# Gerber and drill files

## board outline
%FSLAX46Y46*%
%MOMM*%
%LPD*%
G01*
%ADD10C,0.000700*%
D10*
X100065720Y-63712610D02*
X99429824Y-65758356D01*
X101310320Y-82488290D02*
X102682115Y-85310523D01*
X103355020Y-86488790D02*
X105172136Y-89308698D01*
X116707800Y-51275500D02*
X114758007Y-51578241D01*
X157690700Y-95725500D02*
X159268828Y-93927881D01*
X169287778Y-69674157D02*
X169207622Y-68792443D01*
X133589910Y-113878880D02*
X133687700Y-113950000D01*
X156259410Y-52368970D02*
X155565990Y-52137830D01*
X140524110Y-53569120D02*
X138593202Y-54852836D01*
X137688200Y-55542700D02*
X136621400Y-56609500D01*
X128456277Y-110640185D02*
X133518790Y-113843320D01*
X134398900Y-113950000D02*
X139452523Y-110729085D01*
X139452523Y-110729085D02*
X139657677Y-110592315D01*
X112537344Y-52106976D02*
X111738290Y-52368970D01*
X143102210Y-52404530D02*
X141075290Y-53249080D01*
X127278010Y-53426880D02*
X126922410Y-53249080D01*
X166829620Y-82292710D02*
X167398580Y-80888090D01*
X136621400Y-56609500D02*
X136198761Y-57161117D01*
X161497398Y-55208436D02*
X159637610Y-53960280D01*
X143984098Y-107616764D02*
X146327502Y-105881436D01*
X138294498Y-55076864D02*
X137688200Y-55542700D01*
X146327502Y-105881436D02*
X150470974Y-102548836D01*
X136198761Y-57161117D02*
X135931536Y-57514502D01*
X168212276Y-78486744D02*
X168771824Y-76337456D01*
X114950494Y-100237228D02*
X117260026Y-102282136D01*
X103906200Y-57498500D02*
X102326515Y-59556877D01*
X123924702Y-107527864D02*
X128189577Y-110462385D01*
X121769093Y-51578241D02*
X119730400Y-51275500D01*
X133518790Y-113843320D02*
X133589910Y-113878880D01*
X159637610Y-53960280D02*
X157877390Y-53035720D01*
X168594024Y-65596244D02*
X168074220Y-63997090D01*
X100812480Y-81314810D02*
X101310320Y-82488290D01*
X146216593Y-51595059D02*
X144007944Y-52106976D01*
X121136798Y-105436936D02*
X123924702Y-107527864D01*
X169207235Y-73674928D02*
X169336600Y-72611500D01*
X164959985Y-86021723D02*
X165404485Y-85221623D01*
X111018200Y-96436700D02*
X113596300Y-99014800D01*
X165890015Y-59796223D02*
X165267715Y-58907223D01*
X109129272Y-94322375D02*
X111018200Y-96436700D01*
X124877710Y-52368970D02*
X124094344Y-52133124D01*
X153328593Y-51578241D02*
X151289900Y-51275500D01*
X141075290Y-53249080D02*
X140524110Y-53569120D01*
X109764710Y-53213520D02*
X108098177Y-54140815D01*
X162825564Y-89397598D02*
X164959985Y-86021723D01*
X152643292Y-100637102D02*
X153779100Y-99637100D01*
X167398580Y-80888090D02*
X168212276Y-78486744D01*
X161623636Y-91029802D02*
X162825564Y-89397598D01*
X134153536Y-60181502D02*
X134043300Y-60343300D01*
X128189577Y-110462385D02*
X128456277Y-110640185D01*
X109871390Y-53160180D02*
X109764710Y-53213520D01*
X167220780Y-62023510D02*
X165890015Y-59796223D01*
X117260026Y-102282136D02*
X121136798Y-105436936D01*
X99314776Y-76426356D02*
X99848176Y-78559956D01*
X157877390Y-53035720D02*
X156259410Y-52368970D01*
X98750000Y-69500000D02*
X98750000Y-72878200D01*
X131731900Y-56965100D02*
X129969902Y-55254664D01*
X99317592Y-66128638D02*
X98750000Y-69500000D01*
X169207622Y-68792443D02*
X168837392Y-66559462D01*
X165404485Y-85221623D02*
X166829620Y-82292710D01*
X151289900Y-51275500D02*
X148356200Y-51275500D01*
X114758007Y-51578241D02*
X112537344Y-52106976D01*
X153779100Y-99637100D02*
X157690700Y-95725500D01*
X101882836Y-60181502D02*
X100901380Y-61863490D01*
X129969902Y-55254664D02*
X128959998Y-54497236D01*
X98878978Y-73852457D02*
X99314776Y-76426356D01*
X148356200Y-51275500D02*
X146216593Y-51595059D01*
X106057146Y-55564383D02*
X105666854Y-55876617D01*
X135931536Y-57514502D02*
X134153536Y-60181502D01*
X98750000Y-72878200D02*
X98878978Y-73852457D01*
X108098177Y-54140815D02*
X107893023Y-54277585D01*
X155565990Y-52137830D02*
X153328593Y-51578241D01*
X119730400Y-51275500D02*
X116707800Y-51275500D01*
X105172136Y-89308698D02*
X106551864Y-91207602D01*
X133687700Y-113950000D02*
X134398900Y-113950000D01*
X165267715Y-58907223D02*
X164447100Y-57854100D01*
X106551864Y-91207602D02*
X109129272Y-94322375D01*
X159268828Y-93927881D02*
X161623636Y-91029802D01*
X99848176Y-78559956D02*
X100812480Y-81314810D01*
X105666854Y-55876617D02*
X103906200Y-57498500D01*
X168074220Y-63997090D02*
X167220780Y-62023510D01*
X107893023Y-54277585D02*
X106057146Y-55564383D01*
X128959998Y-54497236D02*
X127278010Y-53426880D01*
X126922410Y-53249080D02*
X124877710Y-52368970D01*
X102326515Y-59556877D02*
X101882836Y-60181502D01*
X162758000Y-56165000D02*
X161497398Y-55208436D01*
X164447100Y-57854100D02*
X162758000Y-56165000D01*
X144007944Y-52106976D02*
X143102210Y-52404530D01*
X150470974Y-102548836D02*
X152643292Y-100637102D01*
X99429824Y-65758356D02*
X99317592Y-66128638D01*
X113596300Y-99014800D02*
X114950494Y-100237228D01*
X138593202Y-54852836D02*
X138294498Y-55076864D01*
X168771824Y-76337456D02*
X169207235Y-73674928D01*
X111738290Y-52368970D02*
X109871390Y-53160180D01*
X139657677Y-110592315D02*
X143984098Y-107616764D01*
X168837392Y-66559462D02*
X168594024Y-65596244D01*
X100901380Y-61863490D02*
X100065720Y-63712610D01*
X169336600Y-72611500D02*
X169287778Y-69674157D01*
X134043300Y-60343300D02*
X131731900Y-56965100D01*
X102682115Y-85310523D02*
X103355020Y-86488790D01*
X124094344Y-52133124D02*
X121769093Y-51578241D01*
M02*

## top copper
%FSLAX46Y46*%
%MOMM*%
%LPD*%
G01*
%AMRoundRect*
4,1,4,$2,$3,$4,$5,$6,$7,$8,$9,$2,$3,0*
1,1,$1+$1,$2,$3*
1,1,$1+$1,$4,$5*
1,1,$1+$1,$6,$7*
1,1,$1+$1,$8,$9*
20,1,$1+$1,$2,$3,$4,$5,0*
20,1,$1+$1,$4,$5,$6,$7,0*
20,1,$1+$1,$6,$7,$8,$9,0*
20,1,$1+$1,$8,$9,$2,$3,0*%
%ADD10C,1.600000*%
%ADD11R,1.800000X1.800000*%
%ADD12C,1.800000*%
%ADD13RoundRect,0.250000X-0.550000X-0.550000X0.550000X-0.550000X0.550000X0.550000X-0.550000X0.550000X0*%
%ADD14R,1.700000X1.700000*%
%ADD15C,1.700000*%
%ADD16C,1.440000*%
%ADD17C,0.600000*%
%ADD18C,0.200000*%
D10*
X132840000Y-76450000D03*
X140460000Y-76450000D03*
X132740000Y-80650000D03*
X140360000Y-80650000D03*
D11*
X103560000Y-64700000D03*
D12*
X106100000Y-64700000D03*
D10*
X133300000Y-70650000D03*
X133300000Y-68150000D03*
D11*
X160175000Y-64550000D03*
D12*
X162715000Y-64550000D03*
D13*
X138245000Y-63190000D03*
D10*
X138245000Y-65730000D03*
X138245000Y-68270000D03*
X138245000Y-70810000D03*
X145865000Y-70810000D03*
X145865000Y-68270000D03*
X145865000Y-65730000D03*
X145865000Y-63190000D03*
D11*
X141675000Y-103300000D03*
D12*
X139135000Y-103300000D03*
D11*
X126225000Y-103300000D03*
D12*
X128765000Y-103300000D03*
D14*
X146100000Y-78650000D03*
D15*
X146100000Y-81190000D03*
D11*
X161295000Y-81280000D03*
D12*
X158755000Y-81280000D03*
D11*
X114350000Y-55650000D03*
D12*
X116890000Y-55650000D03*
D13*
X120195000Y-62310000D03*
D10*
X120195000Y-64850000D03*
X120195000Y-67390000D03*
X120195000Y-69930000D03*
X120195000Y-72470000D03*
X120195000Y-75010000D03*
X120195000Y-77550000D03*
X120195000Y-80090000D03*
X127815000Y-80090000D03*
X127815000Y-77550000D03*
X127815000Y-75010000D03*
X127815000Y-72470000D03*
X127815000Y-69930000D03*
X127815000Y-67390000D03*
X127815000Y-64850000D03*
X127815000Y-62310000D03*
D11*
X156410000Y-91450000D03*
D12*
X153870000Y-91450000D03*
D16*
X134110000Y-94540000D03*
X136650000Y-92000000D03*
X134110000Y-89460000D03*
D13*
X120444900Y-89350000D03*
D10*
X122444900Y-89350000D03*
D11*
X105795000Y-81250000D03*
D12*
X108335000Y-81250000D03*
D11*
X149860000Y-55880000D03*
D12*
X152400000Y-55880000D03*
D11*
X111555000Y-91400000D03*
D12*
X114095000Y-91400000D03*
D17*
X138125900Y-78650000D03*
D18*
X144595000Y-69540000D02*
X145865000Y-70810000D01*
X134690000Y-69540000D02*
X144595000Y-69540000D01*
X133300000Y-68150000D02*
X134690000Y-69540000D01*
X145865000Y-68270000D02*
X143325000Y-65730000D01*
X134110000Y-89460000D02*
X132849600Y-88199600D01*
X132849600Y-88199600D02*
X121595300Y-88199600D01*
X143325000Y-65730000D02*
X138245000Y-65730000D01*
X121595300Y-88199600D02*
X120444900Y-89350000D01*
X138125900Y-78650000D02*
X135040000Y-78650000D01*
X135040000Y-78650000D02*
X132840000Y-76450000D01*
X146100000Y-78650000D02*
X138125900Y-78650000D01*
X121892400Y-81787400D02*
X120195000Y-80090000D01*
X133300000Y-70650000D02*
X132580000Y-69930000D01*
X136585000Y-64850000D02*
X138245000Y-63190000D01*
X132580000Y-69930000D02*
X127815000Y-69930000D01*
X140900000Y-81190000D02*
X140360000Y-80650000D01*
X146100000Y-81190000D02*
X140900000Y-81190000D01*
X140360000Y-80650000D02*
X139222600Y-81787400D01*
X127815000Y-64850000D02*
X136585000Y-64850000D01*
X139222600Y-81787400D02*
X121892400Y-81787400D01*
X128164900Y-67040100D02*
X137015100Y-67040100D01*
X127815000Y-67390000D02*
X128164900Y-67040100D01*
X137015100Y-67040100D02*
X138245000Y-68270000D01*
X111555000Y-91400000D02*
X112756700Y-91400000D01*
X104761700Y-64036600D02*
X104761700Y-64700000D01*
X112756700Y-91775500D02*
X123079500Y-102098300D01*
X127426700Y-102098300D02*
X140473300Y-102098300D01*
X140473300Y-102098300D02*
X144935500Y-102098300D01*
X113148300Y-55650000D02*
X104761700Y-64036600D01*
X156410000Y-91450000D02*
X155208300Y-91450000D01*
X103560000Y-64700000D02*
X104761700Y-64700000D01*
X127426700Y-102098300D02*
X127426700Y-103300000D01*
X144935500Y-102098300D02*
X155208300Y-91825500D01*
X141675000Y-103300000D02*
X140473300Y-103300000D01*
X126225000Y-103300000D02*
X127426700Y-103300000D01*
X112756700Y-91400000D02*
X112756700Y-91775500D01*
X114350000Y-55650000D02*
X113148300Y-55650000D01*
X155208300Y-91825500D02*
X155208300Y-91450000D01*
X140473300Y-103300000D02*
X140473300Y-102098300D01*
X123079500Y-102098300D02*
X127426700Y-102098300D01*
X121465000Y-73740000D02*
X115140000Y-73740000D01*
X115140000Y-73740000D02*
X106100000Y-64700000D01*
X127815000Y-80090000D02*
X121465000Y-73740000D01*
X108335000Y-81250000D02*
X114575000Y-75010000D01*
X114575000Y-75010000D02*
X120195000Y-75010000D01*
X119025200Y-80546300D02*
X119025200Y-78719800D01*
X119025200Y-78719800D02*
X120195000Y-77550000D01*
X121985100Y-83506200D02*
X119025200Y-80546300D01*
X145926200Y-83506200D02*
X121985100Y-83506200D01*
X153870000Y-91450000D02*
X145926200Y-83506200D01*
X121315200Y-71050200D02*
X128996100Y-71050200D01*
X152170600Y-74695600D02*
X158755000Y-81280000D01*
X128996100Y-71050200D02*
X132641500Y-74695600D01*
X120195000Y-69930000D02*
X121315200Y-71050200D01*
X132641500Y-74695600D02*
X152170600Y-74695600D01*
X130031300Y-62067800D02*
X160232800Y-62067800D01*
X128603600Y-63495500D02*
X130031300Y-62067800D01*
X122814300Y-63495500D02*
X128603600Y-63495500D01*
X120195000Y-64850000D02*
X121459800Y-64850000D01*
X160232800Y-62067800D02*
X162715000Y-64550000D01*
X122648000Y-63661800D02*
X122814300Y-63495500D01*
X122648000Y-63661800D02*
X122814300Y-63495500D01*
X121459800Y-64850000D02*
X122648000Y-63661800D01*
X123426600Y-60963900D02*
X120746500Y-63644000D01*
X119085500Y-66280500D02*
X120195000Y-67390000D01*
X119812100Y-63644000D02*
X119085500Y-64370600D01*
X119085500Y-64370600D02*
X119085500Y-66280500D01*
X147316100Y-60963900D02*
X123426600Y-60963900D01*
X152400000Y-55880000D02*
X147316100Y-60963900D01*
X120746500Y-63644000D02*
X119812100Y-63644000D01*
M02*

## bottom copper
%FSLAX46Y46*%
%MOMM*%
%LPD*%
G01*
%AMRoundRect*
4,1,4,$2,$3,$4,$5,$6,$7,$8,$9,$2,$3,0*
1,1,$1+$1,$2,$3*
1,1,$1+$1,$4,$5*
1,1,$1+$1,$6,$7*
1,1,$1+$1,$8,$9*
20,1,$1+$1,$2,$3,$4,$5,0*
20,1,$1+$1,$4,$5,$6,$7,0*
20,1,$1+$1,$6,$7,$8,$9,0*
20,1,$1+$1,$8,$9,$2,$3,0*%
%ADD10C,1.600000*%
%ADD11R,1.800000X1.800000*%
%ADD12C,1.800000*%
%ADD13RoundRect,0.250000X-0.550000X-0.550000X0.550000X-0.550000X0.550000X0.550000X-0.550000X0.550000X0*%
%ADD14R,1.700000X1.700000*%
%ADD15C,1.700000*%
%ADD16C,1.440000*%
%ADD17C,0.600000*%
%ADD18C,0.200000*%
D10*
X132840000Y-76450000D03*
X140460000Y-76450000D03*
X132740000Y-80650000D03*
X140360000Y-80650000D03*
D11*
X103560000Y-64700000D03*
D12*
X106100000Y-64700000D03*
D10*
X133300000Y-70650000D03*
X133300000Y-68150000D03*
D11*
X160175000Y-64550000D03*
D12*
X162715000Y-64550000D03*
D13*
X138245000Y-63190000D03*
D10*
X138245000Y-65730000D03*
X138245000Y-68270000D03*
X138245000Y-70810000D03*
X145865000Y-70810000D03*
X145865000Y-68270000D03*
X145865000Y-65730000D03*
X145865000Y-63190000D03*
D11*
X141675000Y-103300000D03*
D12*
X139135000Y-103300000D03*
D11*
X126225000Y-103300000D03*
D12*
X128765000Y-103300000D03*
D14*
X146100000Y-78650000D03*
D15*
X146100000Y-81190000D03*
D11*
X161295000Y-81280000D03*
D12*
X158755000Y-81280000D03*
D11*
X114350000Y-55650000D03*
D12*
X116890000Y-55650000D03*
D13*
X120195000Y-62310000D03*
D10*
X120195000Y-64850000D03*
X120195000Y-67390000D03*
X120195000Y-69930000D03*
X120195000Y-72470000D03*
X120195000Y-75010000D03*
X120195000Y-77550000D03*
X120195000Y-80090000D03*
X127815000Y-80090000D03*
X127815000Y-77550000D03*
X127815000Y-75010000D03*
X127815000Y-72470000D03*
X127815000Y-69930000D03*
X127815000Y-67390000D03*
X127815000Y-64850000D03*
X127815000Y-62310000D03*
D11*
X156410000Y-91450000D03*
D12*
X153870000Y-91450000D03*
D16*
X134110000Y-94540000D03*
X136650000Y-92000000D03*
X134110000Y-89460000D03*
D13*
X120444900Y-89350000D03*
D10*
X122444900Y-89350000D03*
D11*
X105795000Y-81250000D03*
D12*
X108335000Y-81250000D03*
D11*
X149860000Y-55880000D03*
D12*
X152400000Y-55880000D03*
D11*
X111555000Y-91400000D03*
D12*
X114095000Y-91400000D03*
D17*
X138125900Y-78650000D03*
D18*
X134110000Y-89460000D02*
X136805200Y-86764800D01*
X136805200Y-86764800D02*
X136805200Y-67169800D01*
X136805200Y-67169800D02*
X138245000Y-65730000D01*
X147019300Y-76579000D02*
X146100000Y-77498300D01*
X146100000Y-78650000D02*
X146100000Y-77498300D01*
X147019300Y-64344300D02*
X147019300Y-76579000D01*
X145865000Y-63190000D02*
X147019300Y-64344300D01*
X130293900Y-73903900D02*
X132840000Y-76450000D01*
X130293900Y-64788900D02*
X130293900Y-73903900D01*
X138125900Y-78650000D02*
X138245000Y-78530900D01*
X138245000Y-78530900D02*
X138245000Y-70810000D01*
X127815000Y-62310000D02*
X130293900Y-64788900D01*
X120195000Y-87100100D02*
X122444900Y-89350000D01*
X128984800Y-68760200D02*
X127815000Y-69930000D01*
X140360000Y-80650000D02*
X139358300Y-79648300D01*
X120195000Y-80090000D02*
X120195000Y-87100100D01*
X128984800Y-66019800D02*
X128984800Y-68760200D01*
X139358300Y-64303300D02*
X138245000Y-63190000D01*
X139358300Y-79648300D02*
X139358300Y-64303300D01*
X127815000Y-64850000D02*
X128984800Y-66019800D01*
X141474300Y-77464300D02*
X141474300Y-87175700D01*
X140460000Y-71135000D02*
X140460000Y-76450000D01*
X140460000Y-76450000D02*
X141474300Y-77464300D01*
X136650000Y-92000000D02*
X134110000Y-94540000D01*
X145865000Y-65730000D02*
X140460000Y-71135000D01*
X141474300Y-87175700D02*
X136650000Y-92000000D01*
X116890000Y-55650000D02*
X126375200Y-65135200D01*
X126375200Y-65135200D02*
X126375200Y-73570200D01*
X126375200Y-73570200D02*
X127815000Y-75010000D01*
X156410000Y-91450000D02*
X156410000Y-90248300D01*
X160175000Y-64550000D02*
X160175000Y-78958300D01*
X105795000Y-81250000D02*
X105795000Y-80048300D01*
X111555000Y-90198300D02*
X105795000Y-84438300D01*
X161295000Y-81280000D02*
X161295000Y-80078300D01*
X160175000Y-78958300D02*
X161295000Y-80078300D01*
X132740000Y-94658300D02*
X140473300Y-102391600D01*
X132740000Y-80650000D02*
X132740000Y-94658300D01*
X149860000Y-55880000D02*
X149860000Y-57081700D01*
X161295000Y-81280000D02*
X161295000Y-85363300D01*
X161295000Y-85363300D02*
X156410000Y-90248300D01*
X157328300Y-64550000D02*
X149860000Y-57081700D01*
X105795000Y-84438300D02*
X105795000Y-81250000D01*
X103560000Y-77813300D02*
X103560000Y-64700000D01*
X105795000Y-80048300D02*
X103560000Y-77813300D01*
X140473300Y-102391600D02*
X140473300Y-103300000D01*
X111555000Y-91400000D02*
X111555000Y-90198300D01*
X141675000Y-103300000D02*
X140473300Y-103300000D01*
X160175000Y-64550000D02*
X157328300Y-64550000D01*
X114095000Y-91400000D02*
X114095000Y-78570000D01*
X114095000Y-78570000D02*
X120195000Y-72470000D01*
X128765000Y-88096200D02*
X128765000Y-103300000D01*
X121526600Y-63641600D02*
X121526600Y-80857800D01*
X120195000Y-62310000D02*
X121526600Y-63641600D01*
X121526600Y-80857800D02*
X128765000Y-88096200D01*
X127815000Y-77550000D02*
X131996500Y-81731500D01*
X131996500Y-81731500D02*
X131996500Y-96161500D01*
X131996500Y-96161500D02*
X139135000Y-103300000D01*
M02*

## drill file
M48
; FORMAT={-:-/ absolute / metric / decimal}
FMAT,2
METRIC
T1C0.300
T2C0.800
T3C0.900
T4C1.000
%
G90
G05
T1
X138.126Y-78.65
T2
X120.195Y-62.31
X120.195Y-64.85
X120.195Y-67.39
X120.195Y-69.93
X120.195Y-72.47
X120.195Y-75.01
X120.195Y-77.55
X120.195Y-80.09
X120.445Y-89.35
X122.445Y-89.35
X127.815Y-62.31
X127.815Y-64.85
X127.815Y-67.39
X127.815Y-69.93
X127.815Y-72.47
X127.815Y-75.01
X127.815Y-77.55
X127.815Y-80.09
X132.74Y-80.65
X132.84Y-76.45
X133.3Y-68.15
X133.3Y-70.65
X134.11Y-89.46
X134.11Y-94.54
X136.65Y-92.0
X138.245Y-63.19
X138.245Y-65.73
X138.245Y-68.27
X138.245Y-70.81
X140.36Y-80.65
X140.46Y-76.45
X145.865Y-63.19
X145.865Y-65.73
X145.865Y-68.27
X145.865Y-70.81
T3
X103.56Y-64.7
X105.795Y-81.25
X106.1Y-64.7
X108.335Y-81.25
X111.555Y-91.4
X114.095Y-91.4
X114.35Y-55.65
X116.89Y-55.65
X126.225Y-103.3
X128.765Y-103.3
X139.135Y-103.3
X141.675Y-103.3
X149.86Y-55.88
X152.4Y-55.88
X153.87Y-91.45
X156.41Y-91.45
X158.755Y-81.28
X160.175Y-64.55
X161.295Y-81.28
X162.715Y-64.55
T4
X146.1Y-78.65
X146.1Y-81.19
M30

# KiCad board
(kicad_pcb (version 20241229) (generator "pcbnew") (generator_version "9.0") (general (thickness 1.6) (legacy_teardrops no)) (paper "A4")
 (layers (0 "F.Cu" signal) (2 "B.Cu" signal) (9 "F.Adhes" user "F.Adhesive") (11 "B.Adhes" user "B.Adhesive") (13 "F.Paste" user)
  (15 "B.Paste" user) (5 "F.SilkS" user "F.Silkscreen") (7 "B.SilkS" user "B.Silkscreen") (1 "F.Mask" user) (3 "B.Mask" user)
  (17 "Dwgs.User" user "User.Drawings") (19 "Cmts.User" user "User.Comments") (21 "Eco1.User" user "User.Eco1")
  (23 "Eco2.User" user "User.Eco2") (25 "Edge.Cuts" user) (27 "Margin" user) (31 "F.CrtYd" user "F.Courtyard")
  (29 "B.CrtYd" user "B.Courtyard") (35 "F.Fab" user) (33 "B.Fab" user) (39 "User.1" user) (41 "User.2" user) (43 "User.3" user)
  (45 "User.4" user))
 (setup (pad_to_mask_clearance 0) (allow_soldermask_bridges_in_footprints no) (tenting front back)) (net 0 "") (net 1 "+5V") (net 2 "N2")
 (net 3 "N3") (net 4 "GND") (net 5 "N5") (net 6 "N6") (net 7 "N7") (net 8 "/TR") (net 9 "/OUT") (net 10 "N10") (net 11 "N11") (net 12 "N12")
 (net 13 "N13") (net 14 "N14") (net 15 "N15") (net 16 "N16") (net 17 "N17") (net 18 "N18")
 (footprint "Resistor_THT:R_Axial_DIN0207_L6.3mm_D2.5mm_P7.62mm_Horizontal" (layer "F.Cu") (at 132.84 76.45)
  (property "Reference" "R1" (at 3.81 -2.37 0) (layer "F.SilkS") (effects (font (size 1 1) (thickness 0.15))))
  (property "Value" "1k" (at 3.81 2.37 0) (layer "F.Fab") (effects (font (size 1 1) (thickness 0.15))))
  (pad "1" thru_hole circle (at 0 0) (size 1.6 1.6) (drill 0.8) (layers "*.Cu" "*.Mask") (remove_unused_layers no) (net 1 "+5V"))
  (pad "2" thru_hole circle (at 7.62 0) (size 1.6 1.6) (drill 0.8) (layers "*.Cu" "*.Mask") (remove_unused_layers no) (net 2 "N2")))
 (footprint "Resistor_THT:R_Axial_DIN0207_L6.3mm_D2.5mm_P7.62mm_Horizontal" (layer "F.Cu") (at 132.74 80.65)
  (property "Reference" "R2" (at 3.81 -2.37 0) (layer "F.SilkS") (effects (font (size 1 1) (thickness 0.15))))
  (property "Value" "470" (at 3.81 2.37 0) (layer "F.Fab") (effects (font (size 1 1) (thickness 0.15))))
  (pad "1" thru_hole circle (at 0 0) (size 1.6 1.6) (drill 0.8) (layers "*.Cu" "*.Mask") (remove_unused_layers no) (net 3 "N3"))
  (pad "2" thru_hole circle (at 7.62 0) (size 1.6 1.6) (drill 0.8) (layers "*.Cu" "*.Mask") (remove_unused_layers no) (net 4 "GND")))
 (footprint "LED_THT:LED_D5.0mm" (layer "F.Cu") (at 103.56 64.7)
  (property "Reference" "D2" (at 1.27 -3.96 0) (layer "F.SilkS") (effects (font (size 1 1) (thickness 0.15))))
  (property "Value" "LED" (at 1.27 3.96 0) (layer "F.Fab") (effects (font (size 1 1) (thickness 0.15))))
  (pad "1" thru_hole rect (at 0 0) (size 1.8 1.8) (drill 0.9) (layers "*.Cu" "*.Mask") (remove_unused_layers no) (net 3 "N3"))
  (pad "2" thru_hole circle (at 2.54 0) (size 1.8 1.8) (drill 0.9) (layers "*.Cu" "*.Mask") (remove_unused_layers no) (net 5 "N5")))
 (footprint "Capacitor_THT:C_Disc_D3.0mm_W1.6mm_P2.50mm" (layer "F.Cu") (at 133.3 70.65 90)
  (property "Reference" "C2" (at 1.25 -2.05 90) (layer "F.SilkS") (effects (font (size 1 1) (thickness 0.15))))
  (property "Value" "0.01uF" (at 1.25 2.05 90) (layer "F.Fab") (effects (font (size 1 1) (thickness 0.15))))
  (pad "1" thru_hole circle (at 0 0 90) (size 1.6 1.6) (drill 0.8) (layers "*.Cu" "*.Mask") (remove_unused_layers no) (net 4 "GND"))
  (pad "2" thru_hole circle (at 2.5 0 90) (size 1.6 1.6) (drill 0.8) (layers "*.Cu" "*.Mask") (remove_unused_layers no) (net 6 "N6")))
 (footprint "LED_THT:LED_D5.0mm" (layer "F.Cu") (at 160.175 64.55)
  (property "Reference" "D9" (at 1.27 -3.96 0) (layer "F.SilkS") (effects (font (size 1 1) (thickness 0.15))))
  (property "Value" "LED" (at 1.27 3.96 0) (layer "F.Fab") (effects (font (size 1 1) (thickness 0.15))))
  (pad "1" thru_hole rect (at 0 0) (size 1.8 1.8) (drill 0.9) (layers "*.Cu" "*.Mask") (remove_unused_layers no) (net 3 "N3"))
  (pad "2" thru_hole circle (at 2.54 0) (size 1.8 1.8) (drill 0.9) (layers "*.Cu" "*.Mask") (remove_unused_layers no) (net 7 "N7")))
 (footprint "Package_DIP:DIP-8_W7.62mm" (layer "F.Cu") (at 138.245 63.19)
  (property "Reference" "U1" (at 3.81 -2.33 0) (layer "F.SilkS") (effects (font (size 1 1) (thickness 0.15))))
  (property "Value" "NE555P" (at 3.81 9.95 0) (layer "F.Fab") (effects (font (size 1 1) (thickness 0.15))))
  (pad "1" thru_hole roundrect (at 0 0) (size 1.6 1.6) (drill 0.8) (layers "*.Cu" "*.Mask") (remove_unused_layers no)
   (roundrect_rratio 0.15625) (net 4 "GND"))
  (pad "2" thru_hole circle (at 0 2.54) (size 1.6 1.6) (drill 0.8) (layers "*.Cu" "*.Mask") (remove_unused_layers no) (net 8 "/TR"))
  (pad "3" thru_hole circle (at 0 5.08) (size 1.6 1.6) (drill 0.8) (layers "*.Cu" "*.Mask") (remove_unused_layers no) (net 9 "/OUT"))
  (pad "4" thru_hole circle (at 0 7.62) (size 1.6 1.6) (drill 0.8) (layers "*.Cu" "*.Mask") (remove_unused_layers no) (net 1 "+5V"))
  (pad "5" thru_hole circle (at 7.62 7.62) (size 1.6 1.6) (drill 0.8) (layers "*.Cu" "*.Mask") (remove_unused_layers no) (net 6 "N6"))
  (pad "6" thru_hole circle (at 7.62 5.08) (size 1.6 1.6) (drill 0.8) (layers "*.Cu" "*.Mask") (remove_unused_layers no) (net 8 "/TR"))
  (pad "7" thru_hole circle (at 7.62 2.54) (size 1.6 1.6) (drill 0.8) (layers "*.Cu" "*.Mask") (remove_unused_layers no) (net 2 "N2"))
  (pad "8" thru_hole circle (at 7.62 0) (size 1.6 1.6) (drill 0.8) (layers "*.Cu" "*.Mask") (remove_unused_layers no) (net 1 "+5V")))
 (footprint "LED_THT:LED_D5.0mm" (layer "F.Cu") (at 141.675 103.3 180)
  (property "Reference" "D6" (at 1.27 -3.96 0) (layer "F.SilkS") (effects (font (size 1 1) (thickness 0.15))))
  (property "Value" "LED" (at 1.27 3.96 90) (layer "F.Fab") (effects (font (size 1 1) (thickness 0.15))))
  (pad "1" thru_hole rect (at 0 0 180) (size 1.8 1.8) (drill 0.9) (layers "*.Cu" "*.Mask") (remove_unused_layers no) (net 3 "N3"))
  (pad "2" thru_hole circle (at 2.54 0 180) (size 1.8 1.8) (drill 0.9) (layers "*.Cu" "*.Mask") (remove_unused_layers no) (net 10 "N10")))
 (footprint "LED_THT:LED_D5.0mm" (layer "F.Cu") (at 126.225 103.3)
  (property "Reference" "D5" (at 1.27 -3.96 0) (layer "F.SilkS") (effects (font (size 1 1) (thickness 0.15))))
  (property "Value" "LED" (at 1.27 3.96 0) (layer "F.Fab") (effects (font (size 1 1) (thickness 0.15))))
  (pad "1" thru_hole rect (at 0 0) (size 1.8 1.8) (drill 0.9) (layers "*.Cu" "*.Mask") (remove_unused_layers no) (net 3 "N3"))
  (pad "2" thru_hole circle (at 2.54 0) (size 1.8 1.8) (drill 0.9) (layers "*.Cu" "*.Mask") (remove_unused_layers no) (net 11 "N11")))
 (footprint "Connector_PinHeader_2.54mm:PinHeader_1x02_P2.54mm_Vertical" (layer "F.Cu") (at 146.1 78.65)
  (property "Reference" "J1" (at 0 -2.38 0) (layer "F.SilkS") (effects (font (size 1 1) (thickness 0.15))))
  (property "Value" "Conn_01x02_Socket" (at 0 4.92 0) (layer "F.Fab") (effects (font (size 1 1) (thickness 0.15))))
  (pad "1" thru_hole rect (at 0 0) (size 1.7 1.7) (drill 1) (layers "*.Cu" "*.Mask") (remove_unused_layers no) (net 1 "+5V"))
  (pad "2" thru_hole circle (at 0 2.54) (size 1.7 1.7) (drill 1) (layers "*.Cu" "*.Mask") (remove_unused_layers no) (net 4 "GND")))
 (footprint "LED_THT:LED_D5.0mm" (layer "F.Cu") (at 161.295 81.28 180)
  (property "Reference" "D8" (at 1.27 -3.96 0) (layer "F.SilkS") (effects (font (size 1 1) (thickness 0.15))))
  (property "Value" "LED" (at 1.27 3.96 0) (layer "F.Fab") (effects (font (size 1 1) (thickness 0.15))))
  (pad "1" thru_hole rect (at 0 0 180) (size 1.8 1.8) (drill 0.9) (layers "*.Cu" "*.Mask") (remove_unused_layers no) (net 3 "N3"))
  (pad "2" thru_hole circle (at 2.54 0 180) (size 1.8 1.8) (drill 0.9) (layers "*.Cu" "*.Mask") (remove_unused_layers no) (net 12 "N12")))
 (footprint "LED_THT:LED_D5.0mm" (layer "F.Cu") (at 114.35 55.65)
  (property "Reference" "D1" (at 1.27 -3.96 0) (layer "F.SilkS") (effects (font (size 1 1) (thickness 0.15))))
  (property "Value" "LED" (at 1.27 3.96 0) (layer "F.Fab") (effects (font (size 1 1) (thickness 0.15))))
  (pad "1" thru_hole rect (at 0 0) (size 1.8 1.8) (drill 0.9) (layers "*.Cu" "*.Mask") (remove_unused_layers no) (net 3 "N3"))
  (pad "2" thru_hole circle (at 2.54 0) (size 1.8 1.8) (drill 0.9) (layers "*.Cu" "*.Mask") (remove_unused_layers no) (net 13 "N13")))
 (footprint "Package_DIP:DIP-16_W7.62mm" (layer "F.Cu") (at 120.195 62.31)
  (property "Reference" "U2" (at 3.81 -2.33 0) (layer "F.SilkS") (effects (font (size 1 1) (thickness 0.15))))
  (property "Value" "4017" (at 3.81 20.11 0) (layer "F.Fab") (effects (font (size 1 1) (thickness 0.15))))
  (pad "1" thru_hole roundrect (at 0 0) (size 1.6 1.6) (drill 0.8) (layers "*.Cu" "*.Mask") (remove_unused_layers no)
   (roundrect_rratio 0.15625) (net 11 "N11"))
  (pad "2" thru_hole circle (at 0 2.54) (size 1.6 1.6) (drill 0.8) (layers "*.Cu" "*.Mask") (remove_unused_layers no) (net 7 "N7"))
  (pad "3" thru_hole circle (at 0 5.08) (size 1.6 1.6) (drill 0.8) (layers "*.Cu" "*.Mask") (remove_unused_layers no) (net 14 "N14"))
  (pad "4" thru_hole circle (at 0 7.62) (size 1.6 1.6) (drill 0.8) (layers "*.Cu" "*.Mask") (remove_unused_layers no) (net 12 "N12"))
  (pad "5" thru_hole circle (at 0 10.16) (size 1.6 1.6) (drill 0.8) (layers "*.Cu" "*.Mask") (remove_unused_layers no) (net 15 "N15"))
  (pad "6" thru_hole circle (at 0 12.7) (size 1.6 1.6) (drill 0.8) (layers "*.Cu" "*.Mask") (remove_unused_layers no) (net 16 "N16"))
  (pad "7" thru_hole circle (at 0 15.24) (size 1.6 1.6) (drill 0.8) (layers "*.Cu" "*.Mask") (remove_unused_layers no) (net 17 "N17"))
  (pad "8" thru_hole circle (at 0 17.78) (size 1.6 1.6) (drill 0.8) (layers "*.Cu" "*.Mask") (remove_unused_layers no) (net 4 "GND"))
  (pad "9" thru_hole circle (at 7.62 17.78) (size 1.6 1.6) (drill 0.8) (layers "*.Cu" "*.Mask") (remove_unused_layers no) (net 5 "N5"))
  (pad "10" thru_hole circle (at 7.62 15.24) (size 1.6 1.6) (drill 0.8) (layers "*.Cu" "*.Mask") (remove_unused_layers no) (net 10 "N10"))
  (pad "11" thru_hole circle (at 7.62 12.7) (size 1.6 1.6) (drill 0.8) (layers "*.Cu" "*.Mask") (remove_unused_layers no) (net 13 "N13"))
  (pad "12" thru_hole circle (at 7.62 10.16) (size 1.6 1.6) (drill 0.8) (layers "*.Cu" "*.Mask") (remove_unused_layers no) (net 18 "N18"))
  (pad "13" thru_hole circle (at 7.62 7.62) (size 1.6 1.6) (drill 0.8) (layers "*.Cu" "*.Mask") (remove_unused_layers no) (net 4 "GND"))
  (pad "14" thru_hole circle (at 7.62 5.08) (size 1.6 1.6) (drill 0.8) (layers "*.Cu" "*.Mask") (remove_unused_layers no) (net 9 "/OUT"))
  (pad "15" thru_hole circle (at 7.62 2.54) (size 1.6 1.6) (drill 0.8) (layers "*.Cu" "*.Mask") (remove_unused_layers no) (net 4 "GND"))
  (pad "16" thru_hole circle (at 7.62 0) (size 1.6 1.6) (drill 0.8) (layers "*.Cu" "*.Mask") (remove_unused_layers no) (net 1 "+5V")))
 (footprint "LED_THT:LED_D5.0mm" (layer "F.Cu") (at 156.41 91.45 180)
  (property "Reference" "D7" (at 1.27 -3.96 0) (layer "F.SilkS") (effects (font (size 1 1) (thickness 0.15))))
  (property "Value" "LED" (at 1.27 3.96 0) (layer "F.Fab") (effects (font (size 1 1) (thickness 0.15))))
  (pad "1" thru_hole rect (at 0 0 180) (size 1.8 1.8) (drill 0.9) (layers "*.Cu" "*.Mask") (remove_unused_layers no) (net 3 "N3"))
  (pad "2" thru_hole circle (at 2.54 0 180) (size 1.8 1.8) (drill 0.9) (layers "*.Cu" "*.Mask") (remove_unused_layers no) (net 17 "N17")))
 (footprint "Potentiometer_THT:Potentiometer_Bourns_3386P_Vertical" (layer "F.Cu") (at 134.11 94.54)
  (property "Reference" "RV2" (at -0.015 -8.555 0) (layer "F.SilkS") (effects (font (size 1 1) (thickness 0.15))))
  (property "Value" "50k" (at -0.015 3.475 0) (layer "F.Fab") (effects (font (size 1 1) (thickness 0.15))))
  (pad "1" thru_hole circle (at 0 0) (size 1.44 1.44) (drill 0.8) (layers "*.Cu" "*.Mask") (remove_unused_layers no) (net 2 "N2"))
  (pad "2" thru_hole circle (at 2.54 -2.54) (size 1.44 1.44) (drill 0.8) (layers "*.Cu" "*.Mask") (remove_unused_layers no) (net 2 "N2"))
  (pad "3" thru_hole circle (at 0 -5.08) (size 1.44 1.44) (drill 0.8) (layers "*.Cu" "*.Mask") (remove_unused_layers no) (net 8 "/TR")))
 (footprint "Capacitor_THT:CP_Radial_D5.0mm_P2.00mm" (layer "F.Cu") (at 120.4449 89.35)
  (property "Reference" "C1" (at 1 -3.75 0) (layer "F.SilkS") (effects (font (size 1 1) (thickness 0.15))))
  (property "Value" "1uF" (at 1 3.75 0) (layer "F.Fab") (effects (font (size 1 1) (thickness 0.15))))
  (pad "1" thru_hole roundrect (at 0 0) (size 1.6 1.6) (drill 0.8) (layers "*.Cu" "*.Mask") (remove_unused_layers no)
   (roundrect_rratio 0.15625) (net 8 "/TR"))
  (pad "2" thru_hole circle (at 2 0) (size 1.6 1.6) (drill 0.8) (layers "*.Cu" "*.Mask") (remove_unused_layers no) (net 4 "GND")))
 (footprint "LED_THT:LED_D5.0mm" (layer "F.Cu") (at 105.795 81.25)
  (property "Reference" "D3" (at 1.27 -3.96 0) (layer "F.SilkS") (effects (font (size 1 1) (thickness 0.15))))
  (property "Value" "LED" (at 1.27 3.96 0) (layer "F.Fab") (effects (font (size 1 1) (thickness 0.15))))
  (pad "1" thru_hole rect (at 0 0) (size 1.8 1.8) (drill 0.9) (layers "*.Cu" "*.Mask") (remove_unused_layers no) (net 3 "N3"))
  (pad "2" thru_hole circle (at 2.54 0) (size 1.8 1.8) (drill 0.9) (layers "*.Cu" "*.Mask") (remove_unused_layers no) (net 16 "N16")))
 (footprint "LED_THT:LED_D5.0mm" (layer "F.Cu") (at 149.86 55.88)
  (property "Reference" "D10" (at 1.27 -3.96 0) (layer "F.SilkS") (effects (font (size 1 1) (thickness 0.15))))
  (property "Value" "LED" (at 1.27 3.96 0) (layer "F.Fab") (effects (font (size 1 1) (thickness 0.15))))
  (pad "1" thru_hole rect (at 0 0) (size 1.8 1.8) (drill 0.9) (layers "*.Cu" "*.Mask") (remove_unused_layers no) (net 3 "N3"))
  (pad "2" thru_hole circle (at 2.54 0) (size 1.8 1.8) (drill 0.9) (layers "*.Cu" "*.Mask") (remove_unused_layers no) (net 14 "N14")))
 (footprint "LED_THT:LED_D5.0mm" (layer "F.Cu") (at 111.555 91.4)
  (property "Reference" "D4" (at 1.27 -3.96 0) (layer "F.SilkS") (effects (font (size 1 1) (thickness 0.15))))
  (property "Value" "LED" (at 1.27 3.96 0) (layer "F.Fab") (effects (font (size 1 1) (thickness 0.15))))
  (pad "1" thru_hole rect (at 0 0) (size 1.8 1.8) (drill 0.9) (layers "*.Cu" "*.Mask") (remove_unused_layers no) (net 3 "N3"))
  (pad "2" thru_hole circle (at 2.54 0) (size 1.8 1.8) (drill 0.9) (layers "*.Cu" "*.Mask") (remove_unused_layers no) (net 15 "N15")))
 (gr_line (start 100.06572 63.71261) (end 99.429824 65.758356) (stroke (width 0.0007) (type default)) (layer "Edge.Cuts"))
 (gr_line (start 101.31032 82.48829) (end 102.682115 85.310523) (stroke (width 0.0007) (type default)) (layer "Edge.Cuts"))
 (gr_line (start 103.35502 86.48879) (end 105.172136 89.308698) (stroke (width 0.0007) (type default)) (layer "Edge.Cuts"))
 (gr_line (start 116.7078 51.2755) (end 114.758007 51.578241) (stroke (width 0.0007) (type default)) (layer "Edge.Cuts"))
 (gr_line (start 157.6907 95.7255) (end 159.268828 93.927881) (stroke (width 0.0007) (type default)) (layer "Edge.Cuts"))
 (gr_line (start 169.287778 69.674157) (end 169.207622 68.792443) (stroke (width 0.0007) (type default)) (layer "Edge.Cuts"))
 (gr_line (start 133.58991 113.87888) (end 133.6877 113.95) (stroke (width 0.0007) (type default)) (layer "Edge.Cuts"))
 (gr_line (start 156.25941 52.36897) (end 155.56599 52.13783) (stroke (width 0.0007) (type default)) (layer "Edge.Cuts"))
 (gr_line (start 140.52411 53.56912) (end 138.593202 54.852836) (stroke (width 0.0007) (type default)) (layer "Edge.Cuts"))
 (gr_line (start 137.6882 55.5427) (end 136.6214 56.6095) (stroke (width 0.0007) (type default)) (layer "Edge.Cuts"))
 (gr_line (start 128.456277 110.640185) (end 133.51879 113.84332) (stroke (width 0.0007) (type default)) (layer "Edge.Cuts"))
 (gr_line (start 134.3989 113.95) (end 139.452523 110.729085) (stroke (width 0.0007) (type default)) (layer "Edge.Cuts"))
 (gr_line (start 139.452523 110.729085) (end 139.657677 110.592315) (stroke (width 0.0007) (type default)) (layer "Edge.Cuts"))
 (gr_line (start 112.537344 52.106976) (end 111.73829 52.36897) (stroke (width 0.0007) (type default)) (layer "Edge.Cuts"))
 (gr_line (start 143.10221 52.40453) (end 141.07529 53.24908) (stroke (width 0.0007) (type default)) (layer "Edge.Cuts"))
 (gr_line (start 127.27801 53.42688) (end 126.92241 53.24908) (stroke (width 0.0007) (type default)) (layer "Edge.Cuts"))
 (gr_line (start 166.82962 82.29271) (end 167.39858 80.88809) (stroke (width 0.0007) (type default)) (layer "Edge.Cuts"))
 (gr_line (start 136.6214 56.6095) (end 136.198761 57.161117) (stroke (width 0.0007) (type default)) (layer "Edge.Cuts"))
 (gr_line (start 161.497398 55.208436) (end 159.63761 53.96028) (stroke (width 0.0007) (type default)) (layer "Edge.Cuts"))
 (gr_line (start 143.984098 107.616764) (end 146.327502 105.881436) (stroke (width 0.0007) (type default)) (layer "Edge.Cuts"))
 (gr_line (start 138.294498 55.076864) (end 137.6882 55.5427) (stroke (width 0.0007) (type default)) (layer "Edge.Cuts"))
 (gr_line (start 146.327502 105.881436) (end 150.470974 102.548836) (stroke (width 0.0007) (type default)) (layer "Edge.Cuts"))
 (gr_line (start 136.198761 57.161117) (end 135.931536 57.514502) (stroke (width 0.0007) (type default)) (layer "Edge.Cuts"))
 (gr_line (start 168.212276 78.486744) (end 168.771824 76.337456) (stroke (width 0.0007) (type default)) (layer "Edge.Cuts"))
 (gr_line (start 114.950494 100.237228) (end 117.260026 102.282136) (stroke (width 0.0007) (type default)) (layer "Edge.Cuts"))
 (gr_line (start 103.9062 57.4985) (end 102.326515 59.556877) (stroke (width 0.0007) (type default)) (layer "Edge.Cuts"))
 (gr_line (start 123.924702 107.527864) (end 128.189577 110.462385) (stroke (width 0.0007) (type default)) (layer "Edge.Cuts"))
 (gr_line (start 121.769093 51.578241) (end 119.7304 51.2755) (stroke (width 0.0007) (type default)) (layer "Edge.Cuts"))
 (gr_line (start 133.51879 113.84332) (end 133.58991 113.87888) (stroke (width 0.0007) (type default)) (layer "Edge.Cuts"))
 (gr_line (start 159.63761 53.96028) (end 157.87739 53.03572) (stroke (width 0.0007) (type default)) (layer "Edge.Cuts"))
 (gr_line (start 168.594024 65.596244) (end 168.07422 63.99709) (stroke (width 0.0007) (type default)) (layer "Edge.Cuts"))
 (gr_line (start 100.81248 81.31481) (end 101.31032 82.48829) (stroke (width 0.0007) (type default)) (layer "Edge.Cuts"))
 (gr_line (start 146.216593 51.595059) (end 144.007944 52.106976) (stroke (width 0.0007) (type default)) (layer "Edge.Cuts"))
 (gr_line (start 121.136798 105.436936) (end 123.924702 107.527864) (stroke (width 0.0007) (type default)) (layer "Edge.Cuts"))
 (gr_line (start 169.207235 73.674928) (end 169.3366 72.6115) (stroke (width 0.0007) (type default)) (layer "Edge.Cuts"))
 (gr_line (start 164.959985 86.021723) (end 165.404485 85.221623) (stroke (width 0.0007) (type default)) (layer "Edge.Cuts"))
 (gr_line (start 111.0182 96.4367) (end 113.5963 99.0148) (stroke (width 0.0007) (type default)) (layer "Edge.Cuts"))
 (gr_line (start 165.890015 59.796223) (end 165.267715 58.907223) (stroke (width 0.0007) (type default)) (layer "Edge.Cuts"))
 (gr_line (start 109.129272 94.322375) (end 111.0182 96.4367) (stroke (width 0.0007) (type default)) (layer "Edge.Cuts"))
 (gr_line (start 124.87771 52.36897) (end 124.094344 52.133124) (stroke (width 0.0007) (type default)) (layer "Edge.Cuts"))
 (gr_line (start 153.328593 51.578241) (end 151.2899 51.2755) (stroke (width 0.0007) (type default)) (layer "Edge.Cuts"))
 (gr_line (start 141.07529 53.24908) (end 140.52411 53.56912) (stroke (width 0.0007) (type default)) (layer "Edge.Cuts"))
 (gr_line (start 109.76471 53.21352) (end 108.098177 54.140815) (stroke (width 0.0007) (type default)) (layer "Edge.Cuts"))
 (gr_line (start 162.825564 89.397598) (end 164.959985 86.021723) (stroke (width 0.0007) (type default)) (layer "Edge.Cuts"))
 (gr_line (start 152.643292 100.637102) (end 153.7791 99.6371) (stroke (width 0.0007) (type default)) (layer "Edge.Cuts"))
 (gr_line (start 167.39858 80.88809) (end 168.212276 78.486744) (stroke (width 0.0007) (type default)) (layer "Edge.Cuts"))
 (gr_line (start 161.623636 91.029802) (end 162.825564 89.397598) (stroke (width 0.0007) (type default)) (layer "Edge.Cuts"))
 (gr_line (start 134.153536 60.181502) (end 134.0433 60.3433) (stroke (width 0.0007) (type default)) (layer "Edge.Cuts"))
 (gr_line (start 128.189577 110.462385) (end 128.456277 110.640185) (stroke (width 0.0007) (type default)) (layer "Edge.Cuts"))
 (gr_line (start 109.87139 53.16018) (end 109.76471 53.21352) (stroke (width 0.0007) (type default)) (layer "Edge.Cuts"))
 (gr_line (start 167.22078 62.02351) (end 165.890015 59.796223) (stroke (width 0.0007) (type default)) (layer "Edge.Cuts"))
 (gr_line (start 117.260026 102.282136) (end 121.136798 105.436936) (stroke (width 0.0007) (type default)) (layer "Edge.Cuts"))
 (gr_line (start 99.314776 76.426356) (end 99.848176 78.559956) (stroke (width 0.0007) (type default)) (layer "Edge.Cuts"))
 (gr_line (start 157.87739 53.03572) (end 156.25941 52.36897) (stroke (width 0.0007) (type default)) (layer "Edge.Cuts"))
 (gr_line (start 98.75 69.5) (end 98.75 72.8782) (stroke (width 0.0007) (type default)) (layer "Edge.Cuts"))
 (gr_line (start 131.7319 56.9651) (end 129.969902 55.254664) (stroke (width 0.0007) (type default)) (layer "Edge.Cuts"))
 (gr_line (start 99.317592 66.128638) (end 98.75 69.5) (stroke (width 0.0007) (type default)) (layer "Edge.Cuts"))
 (gr_line (start 169.207622 68.792443) (end 168.837392 66.559462) (stroke (width 0.0007) (type default)) (layer "Edge.Cuts"))
 (gr_line (start 165.404485 85.221623) (end 166.82962 82.29271) (stroke (width 0.0007) (type default)) (layer "Edge.Cuts"))
 (gr_line (start 151.2899 51.2755) (end 148.3562 51.2755) (stroke (width 0.0007) (type default)) (layer "Edge.Cuts"))
 (gr_line (start 114.758007 51.578241) (end 112.537344 52.106976) (stroke (width 0.0007) (type default)) (layer "Edge.Cuts"))
 (gr_line (start 153.7791 99.6371) (end 157.6907 95.7255) (stroke (width 0.0007) (type default)) (layer "Edge.Cuts"))
 (gr_line (start 101.882836 60.181502) (end 100.90138 61.86349) (stroke (width 0.0007) (type default)) (layer "Edge.Cuts"))
 (gr_line (start 129.969902 55.254664) (end 128.959998 54.497236) (stroke (width 0.0007) (type default)) (layer "Edge.Cuts"))
 (gr_line (start 98.878978 73.852457) (end 99.314776 76.426356) (stroke (width 0.0007) (type default)) (layer "Edge.Cuts"))
 (gr_line (start 148.3562 51.2755) (end 146.216593 51.595059) (stroke (width 0.0007) (type default)) (layer "Edge.Cuts"))
 (gr_line (start 106.057146 55.564383) (end 105.666854 55.876617) (stroke (width 0.0007) (type default)) (layer "Edge.Cuts"))
 (gr_line (start 135.931536 57.514502) (end 134.153536 60.181502) (stroke (width 0.0007) (type default)) (layer "Edge.Cuts"))
 (gr_line (start 98.75 72.8782) (end 98.878978 73.852457) (stroke (width 0.0007) (type default)) (layer "Edge.Cuts"))
 (gr_line (start 108.098177 54.140815) (end 107.893023 54.277585) (stroke (width 0.0007) (type default)) (layer "Edge.Cuts"))
 (gr_line (start 155.56599 52.13783) (end 153.328593 51.578241) (stroke (width 0.0007) (type default)) (layer "Edge.Cuts"))
 (gr_line (start 119.7304 51.2755) (end 116.7078 51.2755) (stroke (width 0.0007) (type default)) (layer "Edge.Cuts"))
 (gr_line (start 105.172136 89.308698) (end 106.551864 91.207602) (stroke (width 0.0007) (type default)) (layer "Edge.Cuts"))
 (gr_line (start 133.6877 113.95) (end 134.3989 113.95) (stroke (width 0.0007) (type default)) (layer "Edge.Cuts"))
 (gr_line (start 165.267715 58.907223) (end 164.4471 57.8541) (stroke (width 0.0007) (type default)) (layer "Edge.Cuts"))
 (gr_line (start 106.551864 91.207602) (end 109.129272 94.322375) (stroke (width 0.0007) (type default)) (layer "Edge.Cuts"))
 (gr_line (start 159.268828 93.927881) (end 161.623636 91.029802) (stroke (width 0.0007) (type default)) (layer "Edge.Cuts"))
 (gr_line (start 99.848176 78.559956) (end 100.81248 81.31481) (stroke (width 0.0007) (type default)) (layer "Edge.Cuts"))
 (gr_line (start 105.666854 55.876617) (end 103.9062 57.4985) (stroke (width 0.0007) (type default)) (layer "Edge.Cuts"))
 (gr_line (start 168.07422 63.99709) (end 167.22078 62.02351) (stroke (width 0.0007) (type default)) (layer "Edge.Cuts"))
 (gr_line (start 107.893023 54.277585) (end 106.057146 55.564383) (stroke (width 0.0007) (type default)) (layer "Edge.Cuts"))
 (gr_line (start 128.959998 54.497236) (end 127.27801 53.42688) (stroke (width 0.0007) (type default)) (layer "Edge.Cuts"))
 (gr_line (start 126.92241 53.24908) (end 124.87771 52.36897) (stroke (width 0.0007) (type default)) (layer "Edge.Cuts"))
 (gr_line (start 102.326515 59.556877) (end 101.882836 60.181502) (stroke (width 0.0007) (type default)) (layer "Edge.Cuts"))
 (gr_line (start 162.758 56.165) (end 161.497398 55.208436) (stroke (width 0.0007) (type default)) (layer "Edge.Cuts"))
 (gr_line (start 164.4471 57.8541) (end 162.758 56.165) (stroke (width 0.0007) (type default)) (layer "Edge.Cuts"))
 (gr_line (start 144.007944 52.106976) (end 143.10221 52.40453) (stroke (width 0.0007) (type default)) (layer "Edge.Cuts"))
 (gr_line (start 150.470974 102.548836) (end 152.643292 100.637102) (stroke (width 0.0007) (type default)) (layer "Edge.Cuts"))
 (gr_line (start 99.429824 65.758356) (end 99.317592 66.128638) (stroke (width 0.0007) (type default)) (layer "Edge.Cuts"))
 (gr_line (start 113.5963 99.0148) (end 114.950494 100.237228) (stroke (width 0.0007) (type default)) (layer "Edge.Cuts"))
 (gr_line (start 138.593202 54.852836) (end 138.294498 55.076864) (stroke (width 0.0007) (type default)) (layer "Edge.Cuts"))
 (gr_line (start 168.771824 76.337456) (end 169.207235 73.674928) (stroke (width 0.0007) (type default)) (layer "Edge.Cuts"))
 (gr_line (start 111.73829 52.36897) (end 109.87139 53.16018) (stroke (width 0.0007) (type default)) (layer "Edge.Cuts"))
 (gr_line (start 139.657677 110.592315) (end 143.984098 107.616764) (stroke (width 0.0007) (type default)) (layer "Edge.Cuts"))
 (gr_line (start 168.837392 66.559462) (end 168.594024 65.596244) (stroke (width 0.0007) (type default)) (layer "Edge.Cuts"))
 (gr_line (start 100.90138 61.86349) (end 100.06572 63.71261) (stroke (width 0.0007) (type default)) (layer "Edge.Cuts"))
 (gr_line (start 169.3366 72.6115) (end 169.287778 69.674157) (stroke (width 0.0007) (type default)) (layer "Edge.Cuts"))
 (gr_line (start 134.0433 60.3433) (end 131.7319 56.9651) (stroke (width 0.0007) (type default)) (layer "Edge.Cuts"))
 (gr_line (start 102.682115 85.310523) (end 103.35502 86.48879) (stroke (width 0.0007) (type default)) (layer "Edge.Cuts"))
 (gr_line (start 124.094344 52.133124) (end 121.769093 51.578241) (stroke (width 0.0007) (type default)) (layer "Edge.Cuts"))
 (segment (start 144.595 69.54) (end 145.865 70.81) (width 0.2) (layer "F.Cu") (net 6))
 (segment (start 134.69 69.54) (end 144.595 69.54) (width 0.2) (layer "F.Cu") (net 6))
 (segment (start 133.3 68.15) (end 134.69 69.54) (width 0.2) (layer "F.Cu") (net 6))
 (segment (start 145.865 68.27) (end 143.325 65.73) (width 0.2) (layer "F.Cu") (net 8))
 (segment (start 134.11 89.46) (end 132.8496 88.1996) (width 0.2) (layer "F.Cu") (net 8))
 (segment (start 132.8496 88.1996) (end 121.5953 88.1996) (width 0.2) (layer "F.Cu") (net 8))
 (segment (start 143.325 65.73) (end 138.245 65.73) (width 0.2) (layer "F.Cu") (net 8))
 (segment (start 121.5953 88.1996) (end 120.4449 89.35) (width 0.2) (layer "F.Cu") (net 8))
 (segment (start 134.11 89.46) (end 136.8052 86.7648) (width 0.2) (layer "B.Cu") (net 8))
 (segment (start 136.8052 86.7648) (end 136.8052 67.1698) (width 0.2) (layer "B.Cu") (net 8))
 (segment (start 136.8052 67.1698) (end 138.245 65.73) (width 0.2) (layer "B.Cu") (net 8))
 (segment (start 138.1259 78.65) (end 135.04 78.65) (width 0.2) (layer "F.Cu") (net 1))
 (segment (start 135.04 78.65) (end 132.84 76.45) (width 0.2) (layer "F.Cu") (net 1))
 (segment (start 146.1 78.65) (end 138.1259 78.65) (width 0.2) (layer "F.Cu") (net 1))
 (via (at 138.1259 78.65) (size 0.6) (drill 0.3) (layers "F.Cu" "B.Cu") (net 1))
 (segment (start 147.0193 76.579) (end 146.1 77.4983) (width 0.2) (layer "B.Cu") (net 1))
 (segment (start 146.1 78.65) (end 146.1 77.4983) (width 0.2) (layer "B.Cu") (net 1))
 (segment (start 147.0193 64.3443) (end 147.0193 76.579) (width 0.2) (layer "B.Cu") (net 1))
 (segment (start 145.865 63.19) (end 147.0193 64.3443) (width 0.2) (layer "B.Cu") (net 1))
 (segment (start 130.2939 73.9039) (end 132.84 76.45) (width 0.2) (layer "B.Cu") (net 1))
 (segment (start 130.2939 64.7889) (end 130.2939 73.9039) (width 0.2) (layer "B.Cu") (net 1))
 (segment (start 138.1259 78.65) (end 138.245 78.5309) (width 0.2) (layer "B.Cu") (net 1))
 (segment (start 138.245 78.5309) (end 138.245 70.81) (width 0.2) (layer "B.Cu") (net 1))
 (segment (start 127.815 62.31) (end 130.2939 64.7889) (width 0.2) (layer "B.Cu") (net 1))
 (segment (start 121.8924 81.7874) (end 120.195 80.09) (width 0.2) (layer "F.Cu") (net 4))
 (segment (start 133.3 70.65) (end 132.58 69.93) (width 0.2) (layer "F.Cu") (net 4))
 (segment (start 136.585 64.85) (end 138.245 63.19) (width 0.2) (layer "F.Cu") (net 4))
 (segment (start 132.58 69.93) (end 127.815 69.93) (width 0.2) (layer "F.Cu") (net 4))
 (segment (start 140.9 81.19) (end 140.36 80.65) (width 0.2) (layer "F.Cu") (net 4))
 (segment (start 146.1 81.19) (end 140.9 81.19) (width 0.2) (layer "F.Cu") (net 4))
 (segment (start 140.36 80.65) (end 139.2226 81.7874) (width 0.2) (layer "F.Cu") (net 4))
 (segment (start 127.815 64.85) (end 136.585 64.85) (width 0.2) (layer "F.Cu") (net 4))
 (segment (start 139.2226 81.7874) (end 121.8924 81.7874) (width 0.2) (layer "F.Cu") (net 4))
 (segment (start 120.195 87.1001) (end 122.4449 89.35) (width 0.2) (layer "B.Cu") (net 4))
 (segment (start 128.9848 68.7602) (end 127.815 69.93) (width 0.2) (layer "B.Cu") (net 4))
 (segment (start 140.36 80.65) (end 139.3583 79.6483) (width 0.2) (layer "B.Cu") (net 4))
 (segment (start 120.195 80.09) (end 120.195 87.1001) (width 0.2) (layer "B.Cu") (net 4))
 (segment (start 128.9848 66.0198) (end 128.9848 68.7602) (width 0.2) (layer "B.Cu") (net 4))
 (segment (start 139.3583 64.3033) (end 138.245 63.19) (width 0.2) (layer "B.Cu") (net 4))
 (segment (start 139.3583 79.6483) (end 139.3583 64.3033) (width 0.2) (layer "B.Cu") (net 4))
 (segment (start 127.815 64.85) (end 128.9848 66.0198) (width 0.2) (layer "B.Cu") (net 4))
 (segment (start 141.4743 77.4643) (end 141.4743 87.1757) (width 0.2) (layer "B.Cu") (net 2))
 (segment (start 140.46 71.135) (end 140.46 76.45) (width 0.2) (layer "B.Cu") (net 2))
 (segment (start 140.46 76.45) (end 141.4743 77.4643) (width 0.2) (layer "B.Cu") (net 2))
 (segment (start 136.65 92) (end 134.11 94.54) (width 0.2) (layer "B.Cu") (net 2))
 (segment (start 145.865 65.73) (end 140.46 71.135) (width 0.2) (layer "B.Cu") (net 2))
 (segment (start 141.4743 87.1757) (end 136.65 92) (width 0.2) (layer "B.Cu") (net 2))
 (segment (start 128.1649 67.0401) (end 137.0151 67.0401) (width 0.2) (layer "F.Cu") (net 9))
 (segment (start 127.815 67.39) (end 128.1649 67.0401) (width 0.2) (layer "F.Cu") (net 9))
 (segment (start 137.0151 67.0401) (end 138.245 68.27) (width 0.2) (layer "F.Cu") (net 9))
 (segment (start 116.89 55.65) (end 126.3752 65.1352) (width 0.2) (layer "B.Cu") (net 13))
 (segment (start 126.3752 65.1352) (end 126.3752 73.5702) (width 0.2) (layer "B.Cu") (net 13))
 (segment (start 126.3752 73.5702) (end 127.815 75.01) (width 0.2) (layer "B.Cu") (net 13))
 (segment (start 111.555 91.4) (end 112.7567 91.4) (width 0.2) (layer "F.Cu") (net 3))
 (segment (start 104.7617 64.0366) (end 104.7617 64.7) (width 0.2) (layer "F.Cu") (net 3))
 (segment (start 112.7567 91.7755) (end 123.0795 102.0983) (width 0.2) (layer "F.Cu") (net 3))
 (segment (start 127.4267 102.0983) (end 140.4733 102.0983) (width 0.2) (layer "F.Cu") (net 3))
 (segment (start 140.4733 102.0983) (end 144.9355 102.0983) (width 0.2) (layer "F.Cu") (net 3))
 (segment (start 113.1483 55.65) (end 104.7617 64.0366) (width 0.2) (layer "F.Cu") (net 3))
 (segment (start 156.41 91.45) (end 155.2083 91.45) (width 0.2) (layer "F.Cu") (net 3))
 (segment (start 103.56 64.7) (end 104.7617 64.7) (width 0.2) (layer "F.Cu") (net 3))
 (segment (start 127.4267 102.0983) (end 127.4267 103.3) (width 0.2) (layer "F.Cu") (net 3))
 (segment (start 144.9355 102.0983) (end 155.2083 91.8255) (width 0.2) (layer "F.Cu") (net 3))
 (segment (start 141.675 103.3) (end 140.4733 103.3) (width 0.2) (layer "F.Cu") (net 3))
 (segment (start 126.225 103.3) (end 127.4267 103.3) (width 0.2) (layer "F.Cu") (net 3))
 (segment (start 112.7567 91.4) (end 112.7567 91.7755) (width 0.2) (layer "F.Cu") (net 3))
 (segment (start 114.35 55.65) (end 113.1483 55.65) (width 0.2) (layer "F.Cu") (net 3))
 (segment (start 155.2083 91.8255) (end 155.2083 91.45) (width 0.2) (layer "F.Cu") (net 3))
 (segment (start 140.4733 103.3) (end 140.4733 102.0983) (width 0.2) (layer "F.Cu") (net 3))
 (segment (start 123.0795 102.0983) (end 127.4267 102.0983) (width 0.2) (layer "F.Cu") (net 3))
 (segment (start 156.41 91.45) (end 156.41 90.2483) (width 0.2) (layer "B.Cu") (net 3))
 (segment (start 160.175 64.55) (end 160.175 78.9583) (width 0.2) (layer "B.Cu") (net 3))
 (segment (start 105.795 81.25) (end 105.795 80.0483) (width 0.2) (layer "B.Cu") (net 3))
 (segment (start 111.555 90.1983) (end 105.795 84.4383) (width 0.2) (layer "B.Cu") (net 3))
 (segment (start 161.295 81.28) (end 161.295 80.0783) (width 0.2) (layer "B.Cu") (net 3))
 (segment (start 160.175 78.9583) (end 161.295 80.0783) (width 0.2) (layer "B.Cu") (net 3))
 (segment (start 132.74 94.6583) (end 140.4733 102.3916) (width 0.2) (layer "B.Cu") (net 3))
 (segment (start 132.74 80.65) (end 132.74 94.6583) (width 0.2) (layer "B.Cu") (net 3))
 (segment (start 149.86 55.88) (end 149.86 57.0817) (width 0.2) (layer "B.Cu") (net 3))
 (segment (start 161.295 81.28) (end 161.295 85.3633) (width 0.2) (layer "B.Cu") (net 3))
 (segment (start 161.295 85.3633) (end 156.41 90.2483) (width 0.2) (layer "B.Cu") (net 3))
 (segment (start 157.3283 64.55) (end 149.86 57.0817) (width 0.2) (layer "B.Cu") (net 3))
 (segment (start 105.795 84.4383) (end 105.795 81.25) (width 0.2) (layer "B.Cu") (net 3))
 (segment (start 103.56 77.8133) (end 103.56 64.7) (width 0.2) (layer "B.Cu") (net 3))
 (segment (start 105.795 80.0483) (end 103.56 77.8133) (width 0.2) (layer "B.Cu") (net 3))
 (segment (start 140.4733 102.3916) (end 140.4733 103.3) (width 0.2) (layer "B.Cu") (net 3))
 (segment (start 111.555 91.4) (end 111.555 90.1983) (width 0.2) (layer "B.Cu") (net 3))
 (segment (start 141.675 103.3) (end 140.4733 103.3) (width 0.2) (layer "B.Cu") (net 3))
 (segment (start 160.175 64.55) (end 157.3283 64.55) (width 0.2) (layer "B.Cu") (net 3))
 (segment (start 121.465 73.74) (end 115.14 73.74) (width 0.2) (layer "F.Cu") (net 5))
 (segment (start 115.14 73.74) (end 106.1 64.7) (width 0.2) (layer "F.Cu") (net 5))
 (segment (start 127.815 80.09) (end 121.465 73.74) (width 0.2) (layer "F.Cu") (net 5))
 (segment (start 108.335 81.25) (end 114.575 75.01) (width 0.2) (layer "F.Cu") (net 16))
 (segment (start 114.575 75.01) (end 120.195 75.01) (width 0.2) (layer "F.Cu") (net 16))
 (segment (start 114.095 91.4) (end 114.095 78.57) (width 0.2) (layer "B.Cu") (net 15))
 (segment (start 114.095 78.57) (end 120.195 72.47) (width 0.2) (layer "B.Cu") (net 15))
 (segment (start 128.765 88.0962) (end 128.765 103.3) (width 0.2) (layer "B.Cu") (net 11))
 (segment (start 121.5266 63.6416) (end 121.5266 80.8578) (width 0.2) (layer "B.Cu") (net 11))
 (segment (start 120.195 62.31) (end 121.5266 63.6416) (width 0.2) (layer "B.Cu") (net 11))
 (segment (start 121.5266 80.8578) (end 128.765 88.0962) (width 0.2) (layer "B.Cu") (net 11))
 (segment (start 127.815 77.55) (end 131.9965 81.7315) (width 0.2) (layer "B.Cu") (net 10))
 (segment (start 131.9965 81.7315) (end 131.9965 96.1615) (width 0.2) (layer "B.Cu") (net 10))
 (segment (start 131.9965 96.1615) (end 139.135 103.3) (width 0.2) (layer "B.Cu") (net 10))
 (segment (start 119.0252 80.5463) (end 119.0252 78.7198) (width 0.2) (layer "F.Cu") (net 17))
 (segment (start 119.0252 78.7198) (end 120.195 77.55) (width 0.2) (layer "F.Cu") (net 17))
 (segment (start 121.9851 83.5062) (end 119.0252 80.5463) (width 0.2) (layer "F.Cu") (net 17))
 (segment (start 145.9262 83.5062) (end 121.9851 83.5062) (width 0.2) (layer "F.Cu") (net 17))
 (segment (start 153.87 91.45) (end 145.9262 83.5062) (width 0.2) (layer "F.Cu") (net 17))
 (segment (start 121.3152 71.0502) (end 128.9961 71.0502) (width 0.2) (layer "F.Cu") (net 12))
 (segment (start 152.1706 74.6956) (end 158.755 81.28) (width 0.2) (layer "F.Cu") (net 12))
 (segment (start 128.9961 71.0502) (end 132.6415 74.6956) (width 0.2) (layer "F.Cu") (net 12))
 (segment (start 120.195 69.93) (end 121.3152 71.0502) (width 0.2) (layer "F.Cu") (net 12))
 (segment (start 132.6415 74.6956) (end 152.1706 74.6956) (width 0.2) (layer "F.Cu") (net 12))
 (segment (start 130.0313 62.0678) (end 160.2328 62.0678) (width 0.2) (layer "F.Cu") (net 7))
 (segment (start 128.6036 63.4955) (end 130.0313 62.0678) (width 0.2) (layer "F.Cu") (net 7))
 (segment (start 122.8143 63.4955) (end 128.6036 63.4955) (width 0.2) (layer "F.Cu") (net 7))
 (segment (start 120.195 64.85) (end 121.4598 64.85) (width 0.2) (layer "F.Cu") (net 7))
 (segment (start 160.2328 62.0678) (end 162.715 64.55) (width 0.2) (layer "F.Cu") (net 7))
 (segment (start 122.648 63.6618) (end 122.8143 63.4955) (width 0.2) (layer "F.Cu") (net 7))
 (segment (start 122.648 63.6618) (end 122.8143 63.4955) (width 0.2) (layer "F.Cu") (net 7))
 (segment (start 121.4598 64.85) (end 122.648 63.6618) (width 0.2) (layer "F.Cu") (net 7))
 (segment (start 123.4266 60.9639) (end 120.7465 63.644) (width 0.2) (layer "F.Cu") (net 14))
 (segment (start 119.0855 66.2805) (end 120.195 67.39) (width 0.2) (layer "F.Cu") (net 14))
 (segment (start 119.8121 63.644) (end 119.0855 64.3706) (width 0.2) (layer "F.Cu") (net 14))
 (segment (start 119.0855 64.3706) (end 119.0855 66.2805) (width 0.2) (layer "F.Cu") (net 14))
 (segment (start 147.3161 60.9639) (end 123.4266 60.9639) (width 0.2) (layer "F.Cu") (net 14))
 (segment (start 152.4 55.88) (end 147.3161 60.9639) (width 0.2) (layer "F.Cu") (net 14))
 (segment (start 120.7465 63.644) (end 119.8121 63.644) (width 0.2) (layer "F.Cu") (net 14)))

